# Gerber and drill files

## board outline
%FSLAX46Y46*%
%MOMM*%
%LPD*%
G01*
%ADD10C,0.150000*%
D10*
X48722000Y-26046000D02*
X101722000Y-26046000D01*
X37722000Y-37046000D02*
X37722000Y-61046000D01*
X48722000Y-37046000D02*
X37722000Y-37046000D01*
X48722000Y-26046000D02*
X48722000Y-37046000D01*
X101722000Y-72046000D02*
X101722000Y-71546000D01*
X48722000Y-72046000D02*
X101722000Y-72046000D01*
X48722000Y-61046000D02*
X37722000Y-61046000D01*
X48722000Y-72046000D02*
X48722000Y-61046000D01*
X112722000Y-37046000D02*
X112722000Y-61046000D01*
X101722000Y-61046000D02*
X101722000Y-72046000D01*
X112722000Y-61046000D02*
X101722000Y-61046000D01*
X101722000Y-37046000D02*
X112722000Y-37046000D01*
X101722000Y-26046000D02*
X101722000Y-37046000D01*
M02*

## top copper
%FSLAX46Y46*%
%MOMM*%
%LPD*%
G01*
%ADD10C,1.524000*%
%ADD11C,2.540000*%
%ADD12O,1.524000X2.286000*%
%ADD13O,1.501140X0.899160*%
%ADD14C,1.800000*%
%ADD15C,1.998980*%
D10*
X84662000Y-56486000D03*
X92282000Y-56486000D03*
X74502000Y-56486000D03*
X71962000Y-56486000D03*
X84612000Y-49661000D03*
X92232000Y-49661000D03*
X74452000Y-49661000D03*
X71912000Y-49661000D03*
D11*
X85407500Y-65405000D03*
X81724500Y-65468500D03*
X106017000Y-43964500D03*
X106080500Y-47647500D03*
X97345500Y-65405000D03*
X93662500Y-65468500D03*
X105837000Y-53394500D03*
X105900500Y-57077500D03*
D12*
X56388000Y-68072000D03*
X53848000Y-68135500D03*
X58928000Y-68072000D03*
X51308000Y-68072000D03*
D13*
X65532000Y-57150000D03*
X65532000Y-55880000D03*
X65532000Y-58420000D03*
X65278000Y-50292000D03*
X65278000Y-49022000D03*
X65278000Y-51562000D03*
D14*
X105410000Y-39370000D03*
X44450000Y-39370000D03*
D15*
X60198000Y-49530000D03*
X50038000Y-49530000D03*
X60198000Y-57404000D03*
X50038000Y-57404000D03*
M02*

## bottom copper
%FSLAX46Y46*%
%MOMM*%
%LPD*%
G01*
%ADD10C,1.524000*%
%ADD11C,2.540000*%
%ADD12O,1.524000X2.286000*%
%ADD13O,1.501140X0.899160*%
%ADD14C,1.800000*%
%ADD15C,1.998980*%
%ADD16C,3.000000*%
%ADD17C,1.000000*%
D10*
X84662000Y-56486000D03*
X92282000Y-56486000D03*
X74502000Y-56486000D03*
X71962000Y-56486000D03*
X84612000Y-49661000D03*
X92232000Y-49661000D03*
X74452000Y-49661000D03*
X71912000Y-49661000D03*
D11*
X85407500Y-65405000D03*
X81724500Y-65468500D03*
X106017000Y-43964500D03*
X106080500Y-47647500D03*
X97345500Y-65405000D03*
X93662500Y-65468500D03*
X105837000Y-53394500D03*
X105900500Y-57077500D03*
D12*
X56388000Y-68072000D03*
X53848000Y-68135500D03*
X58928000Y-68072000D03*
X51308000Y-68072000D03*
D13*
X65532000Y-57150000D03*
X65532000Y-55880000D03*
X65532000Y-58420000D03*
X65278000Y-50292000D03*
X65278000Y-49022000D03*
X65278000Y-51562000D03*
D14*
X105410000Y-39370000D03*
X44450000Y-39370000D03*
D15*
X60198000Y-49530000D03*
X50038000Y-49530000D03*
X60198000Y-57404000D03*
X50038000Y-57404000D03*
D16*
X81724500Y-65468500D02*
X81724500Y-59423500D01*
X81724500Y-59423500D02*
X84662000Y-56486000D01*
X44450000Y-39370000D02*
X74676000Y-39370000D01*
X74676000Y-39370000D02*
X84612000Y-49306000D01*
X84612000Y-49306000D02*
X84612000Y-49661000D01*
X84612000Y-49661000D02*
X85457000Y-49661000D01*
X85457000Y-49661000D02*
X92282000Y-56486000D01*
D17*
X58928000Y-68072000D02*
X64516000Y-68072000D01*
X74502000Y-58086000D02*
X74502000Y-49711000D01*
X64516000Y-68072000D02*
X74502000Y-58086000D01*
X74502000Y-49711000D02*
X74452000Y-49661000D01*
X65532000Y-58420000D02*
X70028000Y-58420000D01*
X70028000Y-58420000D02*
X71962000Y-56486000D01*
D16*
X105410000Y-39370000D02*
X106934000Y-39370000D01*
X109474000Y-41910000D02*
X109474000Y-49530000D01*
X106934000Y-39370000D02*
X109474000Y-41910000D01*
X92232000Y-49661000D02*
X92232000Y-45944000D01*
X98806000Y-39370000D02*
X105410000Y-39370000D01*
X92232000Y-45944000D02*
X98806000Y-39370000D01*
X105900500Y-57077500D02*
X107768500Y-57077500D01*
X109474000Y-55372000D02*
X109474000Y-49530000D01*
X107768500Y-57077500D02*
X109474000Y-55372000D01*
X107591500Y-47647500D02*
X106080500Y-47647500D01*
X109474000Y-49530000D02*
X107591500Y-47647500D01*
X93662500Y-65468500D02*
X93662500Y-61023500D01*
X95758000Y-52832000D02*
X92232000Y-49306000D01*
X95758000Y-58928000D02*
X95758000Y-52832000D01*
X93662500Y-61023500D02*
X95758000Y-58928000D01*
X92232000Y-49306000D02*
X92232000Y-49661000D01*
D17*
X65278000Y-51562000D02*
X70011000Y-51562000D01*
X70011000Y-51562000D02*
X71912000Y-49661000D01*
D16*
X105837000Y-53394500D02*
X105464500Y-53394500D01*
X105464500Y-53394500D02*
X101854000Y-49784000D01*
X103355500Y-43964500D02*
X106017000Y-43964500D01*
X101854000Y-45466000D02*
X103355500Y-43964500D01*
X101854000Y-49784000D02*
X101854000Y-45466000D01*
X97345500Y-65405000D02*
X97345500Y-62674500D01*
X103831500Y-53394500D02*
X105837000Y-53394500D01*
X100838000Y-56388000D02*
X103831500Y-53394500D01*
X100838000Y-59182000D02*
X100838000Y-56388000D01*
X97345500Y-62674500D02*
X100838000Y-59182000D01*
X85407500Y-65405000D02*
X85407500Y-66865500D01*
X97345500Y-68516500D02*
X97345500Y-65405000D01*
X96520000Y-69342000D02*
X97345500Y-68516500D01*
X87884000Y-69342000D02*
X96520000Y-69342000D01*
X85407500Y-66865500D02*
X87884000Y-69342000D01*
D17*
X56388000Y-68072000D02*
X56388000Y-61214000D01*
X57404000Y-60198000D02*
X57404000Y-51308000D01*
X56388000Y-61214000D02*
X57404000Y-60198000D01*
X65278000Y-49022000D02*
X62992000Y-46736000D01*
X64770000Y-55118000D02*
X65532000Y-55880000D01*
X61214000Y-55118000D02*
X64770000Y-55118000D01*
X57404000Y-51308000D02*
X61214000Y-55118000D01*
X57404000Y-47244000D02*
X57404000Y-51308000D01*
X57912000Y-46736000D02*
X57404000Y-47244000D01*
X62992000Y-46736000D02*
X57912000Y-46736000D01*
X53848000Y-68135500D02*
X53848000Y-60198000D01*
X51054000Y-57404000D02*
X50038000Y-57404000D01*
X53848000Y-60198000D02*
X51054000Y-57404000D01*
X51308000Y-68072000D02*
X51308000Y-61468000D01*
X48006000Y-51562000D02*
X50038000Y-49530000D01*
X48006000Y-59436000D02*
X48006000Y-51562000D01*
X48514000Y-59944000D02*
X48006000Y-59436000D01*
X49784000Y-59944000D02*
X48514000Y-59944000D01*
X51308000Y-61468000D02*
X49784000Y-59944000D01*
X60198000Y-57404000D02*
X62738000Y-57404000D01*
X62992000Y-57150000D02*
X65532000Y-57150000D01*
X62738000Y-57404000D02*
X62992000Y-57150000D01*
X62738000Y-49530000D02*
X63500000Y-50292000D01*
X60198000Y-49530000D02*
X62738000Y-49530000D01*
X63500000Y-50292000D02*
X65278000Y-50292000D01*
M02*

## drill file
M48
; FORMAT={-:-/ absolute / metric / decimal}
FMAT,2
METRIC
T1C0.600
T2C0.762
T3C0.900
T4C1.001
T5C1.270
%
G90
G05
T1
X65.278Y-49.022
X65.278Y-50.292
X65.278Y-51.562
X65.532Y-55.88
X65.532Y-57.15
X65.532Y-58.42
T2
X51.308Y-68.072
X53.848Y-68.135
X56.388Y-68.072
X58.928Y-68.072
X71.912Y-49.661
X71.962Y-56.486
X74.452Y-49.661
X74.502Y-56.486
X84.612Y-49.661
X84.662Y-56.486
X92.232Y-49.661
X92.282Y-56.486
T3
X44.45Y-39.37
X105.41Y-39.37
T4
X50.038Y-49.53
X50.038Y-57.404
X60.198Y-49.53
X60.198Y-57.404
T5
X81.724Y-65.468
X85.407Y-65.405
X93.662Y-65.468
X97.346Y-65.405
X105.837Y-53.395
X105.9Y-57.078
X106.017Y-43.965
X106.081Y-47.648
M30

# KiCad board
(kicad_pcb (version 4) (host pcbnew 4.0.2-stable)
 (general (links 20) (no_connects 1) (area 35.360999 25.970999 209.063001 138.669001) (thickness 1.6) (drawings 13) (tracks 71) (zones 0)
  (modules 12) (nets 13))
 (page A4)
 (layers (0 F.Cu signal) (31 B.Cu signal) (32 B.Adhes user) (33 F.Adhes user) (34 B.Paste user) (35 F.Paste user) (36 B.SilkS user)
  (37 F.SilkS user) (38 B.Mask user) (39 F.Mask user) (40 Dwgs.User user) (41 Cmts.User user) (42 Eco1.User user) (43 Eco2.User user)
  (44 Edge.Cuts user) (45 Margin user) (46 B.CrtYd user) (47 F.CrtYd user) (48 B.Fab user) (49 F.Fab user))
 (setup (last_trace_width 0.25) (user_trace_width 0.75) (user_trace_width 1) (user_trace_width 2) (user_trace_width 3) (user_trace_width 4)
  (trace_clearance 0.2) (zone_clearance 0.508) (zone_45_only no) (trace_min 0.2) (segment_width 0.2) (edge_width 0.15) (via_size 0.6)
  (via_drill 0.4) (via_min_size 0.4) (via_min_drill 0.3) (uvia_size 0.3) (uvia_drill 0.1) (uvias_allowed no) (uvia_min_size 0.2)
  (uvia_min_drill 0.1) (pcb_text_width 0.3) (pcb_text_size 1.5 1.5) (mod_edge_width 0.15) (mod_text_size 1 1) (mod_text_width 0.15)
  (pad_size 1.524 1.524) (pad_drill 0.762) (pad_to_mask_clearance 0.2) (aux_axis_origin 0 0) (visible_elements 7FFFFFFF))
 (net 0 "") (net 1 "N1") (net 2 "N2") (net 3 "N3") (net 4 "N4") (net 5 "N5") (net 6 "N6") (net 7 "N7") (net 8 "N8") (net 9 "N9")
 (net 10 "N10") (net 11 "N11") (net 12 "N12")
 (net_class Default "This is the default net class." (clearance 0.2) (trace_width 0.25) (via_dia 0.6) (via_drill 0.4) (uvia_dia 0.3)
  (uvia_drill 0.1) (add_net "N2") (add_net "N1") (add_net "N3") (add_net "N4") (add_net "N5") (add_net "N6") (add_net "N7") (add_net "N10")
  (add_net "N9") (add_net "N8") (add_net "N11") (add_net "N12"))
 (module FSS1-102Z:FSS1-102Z (layer F.Cu) (at 82.122 57.121 180)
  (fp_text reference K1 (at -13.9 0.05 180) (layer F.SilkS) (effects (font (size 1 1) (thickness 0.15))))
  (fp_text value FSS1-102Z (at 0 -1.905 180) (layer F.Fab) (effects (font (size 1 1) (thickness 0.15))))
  (pad 2 thru_hole circle (at -2.54 0.635 180) (size 1.524 1.524) (drill 0.762) (layers *.Cu *.Mask F.SilkS) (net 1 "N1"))
  (pad 1 thru_hole circle (at -10.16 0.635 180) (size 1.524 1.524) (drill 0.762) (layers *.Cu *.Mask F.SilkS) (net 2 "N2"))
  (pad 3 thru_hole circle (at 7.62 0.635 180) (size 1.524 1.524) (drill 0.762) (layers *.Cu *.Mask F.SilkS) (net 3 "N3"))
  (pad 4 thru_hole circle (at 10.16 0.635 180) (size 1.524 1.524) (drill 0.762) (layers *.Cu *.Mask F.SilkS) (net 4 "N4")))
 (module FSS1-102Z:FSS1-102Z (layer F.Cu) (at 82.072 50.296 180)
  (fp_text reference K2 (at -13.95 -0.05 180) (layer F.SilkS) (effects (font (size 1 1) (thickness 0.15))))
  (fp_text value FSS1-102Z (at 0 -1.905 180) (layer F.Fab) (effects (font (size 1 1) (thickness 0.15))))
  (pad 2 thru_hole circle (at -2.54 0.635 180) (size 1.524 1.524) (drill 0.762) (layers *.Cu *.Mask F.SilkS) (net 2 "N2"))
  (pad 1 thru_hole circle (at -10.16 0.635 180) (size 1.524 1.524) (drill 0.762) (layers *.Cu *.Mask F.SilkS) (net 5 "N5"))
  (pad 3 thru_hole circle (at 7.62 0.635 180) (size 1.524 1.524) (drill 0.762) (layers *.Cu *.Mask F.SilkS) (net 3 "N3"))
  (pad 4 thru_hole circle (at 10.16 0.635 180) (size 1.524 1.524) (drill 0.762) (layers *.Cu *.Mask F.SilkS) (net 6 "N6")))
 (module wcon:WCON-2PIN (layer F.Cu) (at 83.566 66.04)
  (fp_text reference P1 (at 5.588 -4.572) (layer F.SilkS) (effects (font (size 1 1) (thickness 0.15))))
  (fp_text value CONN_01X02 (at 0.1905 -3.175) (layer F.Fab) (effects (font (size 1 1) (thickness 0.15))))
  (pad 2 thru_hole circle (at 1.8415 -0.635) (size 2.54 2.54) (drill 1.27) (layers *.Cu *.Mask F.SilkS) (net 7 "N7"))
  (pad 1 thru_hole circle (at -1.8415 -0.5715) (size 2.54 2.54) (drill 1.27) (layers *.Cu *.Mask F.SilkS) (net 1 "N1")))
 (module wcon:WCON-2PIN (layer F.Cu) (at 106.652 45.806 90)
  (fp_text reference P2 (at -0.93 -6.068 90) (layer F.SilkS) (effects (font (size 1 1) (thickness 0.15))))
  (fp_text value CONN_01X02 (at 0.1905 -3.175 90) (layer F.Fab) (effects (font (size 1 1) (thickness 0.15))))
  (pad 2 thru_hole circle (at 1.8415 -0.635 90) (size 2.54 2.54) (drill 1.27) (layers *.Cu *.Mask F.SilkS) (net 7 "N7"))
  (pad 1 thru_hole circle (at -1.8415 -0.5715 90) (size 2.54 2.54) (drill 1.27) (layers *.Cu *.Mask F.SilkS) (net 5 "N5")))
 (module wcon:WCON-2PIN (layer F.Cu) (at 95.504 66.04)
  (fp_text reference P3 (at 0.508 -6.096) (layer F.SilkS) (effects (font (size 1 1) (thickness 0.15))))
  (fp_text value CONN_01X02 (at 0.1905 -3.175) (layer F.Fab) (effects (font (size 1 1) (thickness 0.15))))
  (pad 2 thru_hole circle (at 1.8415 -0.635) (size 2.54 2.54) (drill 1.27) (layers *.Cu *.Mask F.SilkS) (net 7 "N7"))
  (pad 1 thru_hole circle (at -1.8415 -0.5715) (size 2.54 2.54) (drill 1.27) (layers *.Cu *.Mask F.SilkS) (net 5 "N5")))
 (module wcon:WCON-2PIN (layer F.Cu) (at 106.472 55.236 90)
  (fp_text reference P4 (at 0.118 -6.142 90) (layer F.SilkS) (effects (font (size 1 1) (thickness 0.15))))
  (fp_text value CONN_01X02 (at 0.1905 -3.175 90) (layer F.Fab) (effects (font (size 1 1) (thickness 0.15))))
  (pad 2 thru_hole circle (at 1.8415 -0.635 90) (size 2.54 2.54) (drill 1.27) (layers *.Cu *.Mask F.SilkS) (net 7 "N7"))
  (pad 1 thru_hole circle (at -1.8415 -0.5715 90) (size 2.54 2.54) (drill 1.27) (layers *.Cu *.Mask F.SilkS) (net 5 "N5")))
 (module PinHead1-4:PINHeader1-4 (layer F.Cu) (at 55.118 68.072)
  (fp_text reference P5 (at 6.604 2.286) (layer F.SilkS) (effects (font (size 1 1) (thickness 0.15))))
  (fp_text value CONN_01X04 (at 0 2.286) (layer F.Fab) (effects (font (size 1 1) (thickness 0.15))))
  (pad 3 thru_hole oval (at 1.27 0) (size 1.524 2.286) (drill 0.762) (layers *.Cu *.Mask F.SilkS) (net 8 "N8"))
  (pad 2 thru_hole oval (at -1.27 0.0635) (size 1.524 2.286) (drill 0.762) (layers *.Cu *.Mask F.SilkS) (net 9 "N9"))
  (pad 4 thru_hole oval (at 3.81 0) (size 1.524 2.286) (drill 0.762) (layers *.Cu *.Mask F.SilkS) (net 3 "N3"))
  (pad 1 thru_hole oval (at -3.81 0) (size 1.524 2.286) (drill 0.762) (layers *.Cu *.Mask F.SilkS) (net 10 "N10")))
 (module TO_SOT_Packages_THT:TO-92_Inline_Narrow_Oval (layer F.Cu) (at 65.532 58.42 90)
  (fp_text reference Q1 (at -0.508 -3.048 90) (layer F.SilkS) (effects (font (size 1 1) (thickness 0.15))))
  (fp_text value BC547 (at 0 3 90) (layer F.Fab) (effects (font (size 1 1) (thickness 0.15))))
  (pad 2 thru_hole oval (at 1.27 0 270) (size 0.89916 1.50114) (drill 0.6) (layers *.Cu *.Mask F.SilkS) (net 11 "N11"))
  (pad 3 thru_hole oval (at 2.54 0 270) (size 0.89916 1.50114) (drill 0.6) (layers *.Cu *.Mask F.SilkS) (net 8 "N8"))
  (pad 1 thru_hole oval (at 0 0 270) (size 0.89916 1.50114) (drill 0.6) (layers *.Cu *.Mask F.SilkS) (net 4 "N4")))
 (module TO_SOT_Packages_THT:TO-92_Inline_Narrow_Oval (layer F.Cu) (at 65.278 51.562 90)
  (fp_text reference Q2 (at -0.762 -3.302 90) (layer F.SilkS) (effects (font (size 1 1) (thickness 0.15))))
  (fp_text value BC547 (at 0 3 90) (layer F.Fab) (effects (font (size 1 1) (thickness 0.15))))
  (pad 2 thru_hole oval (at 1.27 0 270) (size 0.89916 1.50114) (drill 0.6) (layers *.Cu *.Mask F.SilkS) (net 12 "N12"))
  (pad 3 thru_hole oval (at 2.54 0 270) (size 0.89916 1.50114) (drill 0.6) (layers *.Cu *.Mask F.SilkS) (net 8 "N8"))
  (pad 1 thru_hole oval (at 0 0 270) (size 0.89916 1.50114) (drill 0.6) (layers *.Cu *.Mask F.SilkS) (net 6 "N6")))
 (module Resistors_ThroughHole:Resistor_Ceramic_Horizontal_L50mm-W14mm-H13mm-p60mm (layer F.Cu) (at 74.93 39.37 180)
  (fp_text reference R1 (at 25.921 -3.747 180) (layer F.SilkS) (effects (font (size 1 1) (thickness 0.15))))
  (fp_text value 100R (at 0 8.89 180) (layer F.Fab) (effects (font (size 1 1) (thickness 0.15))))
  (pad 1 thru_hole circle (at -30.48 0) (size 1.8 1.8) (drill 0.9) (layers *.Cu *.Mask F.SilkS) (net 5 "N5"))
  (pad 2 thru_hole circle (at 30.48 0) (size 1.8 1.8) (drill 0.9) (layers *.Cu *.Mask F.SilkS) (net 2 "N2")))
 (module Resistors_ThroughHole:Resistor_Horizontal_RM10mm (layer F.Cu) (at 60.198 49.53 180)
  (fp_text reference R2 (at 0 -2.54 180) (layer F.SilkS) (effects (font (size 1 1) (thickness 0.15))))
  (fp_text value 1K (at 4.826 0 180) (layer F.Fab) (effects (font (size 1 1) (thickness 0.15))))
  (pad 1 thru_hole circle (at 0 0 180) (size 1.99898 1.99898) (drill 1.00076) (layers *.Cu *.SilkS *.Mask) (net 12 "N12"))
  (pad 2 thru_hole circle (at 10.16 0 180) (size 1.99898 1.99898) (drill 1.00076) (layers *.Cu *.SilkS *.Mask) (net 10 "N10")))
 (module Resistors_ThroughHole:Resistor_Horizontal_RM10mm (layer F.Cu) (at 60.198 57.404 180)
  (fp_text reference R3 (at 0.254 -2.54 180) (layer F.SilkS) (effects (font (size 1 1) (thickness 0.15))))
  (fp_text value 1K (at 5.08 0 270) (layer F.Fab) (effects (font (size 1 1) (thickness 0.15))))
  (pad 1 thru_hole circle (at 0 0 180) (size 1.99898 1.99898) (drill 1.00076) (layers *.Cu *.SilkS *.Mask) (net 11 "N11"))
  (pad 2 thru_hole circle (at 10.16 0 180) (size 1.99898 1.99898) (drill 1.00076) (layers *.Cu *.SilkS *.Mask) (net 9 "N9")))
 (gr_line (start 48.722 26.046) (end 101.722 26.046) (angle 90) (layer Edge.Cuts) (width 0.15))
 (gr_line (start 37.722 37.046) (end 37.722 61.046) (angle 90) (layer Edge.Cuts) (width 0.15))
 (gr_line (start 48.722 37.046) (end 37.722 37.046) (angle 90) (layer Edge.Cuts) (width 0.15))
 (gr_line (start 48.722 26.046) (end 48.722 37.046) (angle 90) (layer Edge.Cuts) (width 0.15))
 (gr_line (start 101.722 72.046) (end 101.722 71.546) (angle 90) (layer Edge.Cuts) (width 0.15))
 (gr_line (start 48.722 72.046) (end 101.722 72.046) (angle 90) (layer Edge.Cuts) (width 0.15))
 (gr_line (start 48.722 61.046) (end 37.722 61.046) (angle 90) (layer Edge.Cuts) (width 0.15))
 (gr_line (start 48.722 72.046) (end 48.722 61.046) (angle 90) (layer Edge.Cuts) (width 0.15))
 (gr_line (start 112.722 37.046) (end 112.722 61.046) (angle 90) (layer Edge.Cuts) (width 0.15))
 (gr_line (start 101.722 61.046) (end 101.722 72.046) (angle 90) (layer Edge.Cuts) (width 0.15))
 (gr_line (start 112.722 61.046) (end 101.722 61.046) (angle 90) (layer Edge.Cuts) (width 0.15))
 (gr_line (start 101.722 37.046) (end 112.722 37.046) (angle 90) (layer Edge.Cuts) (width 0.15))
 (gr_line (start 101.722 26.046) (end 101.722 37.046) (angle 90) (layer Edge.Cuts) (width 0.15))
 (segment (start 81.7245 65.4685) (end 81.7245 59.4235) (width 3) (layer B.Cu) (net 1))
 (segment (start 81.7245 59.4235) (end 84.662 56.486) (width 3) (layer B.Cu) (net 1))
 (segment (start 44.45 39.37) (end 74.676 39.37) (width 3) (layer B.Cu) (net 2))
 (segment (start 74.676 39.37) (end 84.612 49.306) (width 3) (layer B.Cu) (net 2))
 (segment (start 84.612 49.306) (end 84.612 49.661) (width 3) (layer B.Cu) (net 2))
 (segment (start 84.612 49.661) (end 85.457 49.661) (width 3) (layer B.Cu) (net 2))
 (segment (start 85.457 49.661) (end 92.282 56.486) (width 3) (layer B.Cu) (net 2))
 (segment (start 58.928 68.072) (end 64.516 68.072) (width 1) (layer B.Cu) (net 3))
 (segment (start 74.502 58.086) (end 74.502 49.711) (width 1) (layer B.Cu) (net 3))
 (segment (start 64.516 68.072) (end 74.502 58.086) (width 1) (layer B.Cu) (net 3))
 (segment (start 74.502 49.711) (end 74.452 49.661) (width 1) (layer B.Cu) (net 3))
 (segment (start 65.532 58.42) (end 70.028 58.42) (width 1) (layer B.Cu) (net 4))
 (segment (start 70.028 58.42) (end 71.962 56.486) (width 1) (layer B.Cu) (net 4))
 (segment (start 105.41 39.37) (end 106.934 39.37) (width 3) (layer B.Cu) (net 5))
 (segment (start 109.474 41.91) (end 109.474 49.53) (width 3) (layer B.Cu) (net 5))
 (segment (start 106.934 39.37) (end 109.474 41.91) (width 3) (layer B.Cu) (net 5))
 (segment (start 92.232 49.661) (end 92.232 45.944) (width 3) (layer B.Cu) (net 5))
 (segment (start 98.806 39.37) (end 105.41 39.37) (width 3) (layer B.Cu) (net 5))
 (segment (start 92.232 45.944) (end 98.806 39.37) (width 3) (layer B.Cu) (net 5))
 (segment (start 105.9005 57.0775) (end 107.7685 57.0775) (width 3) (layer B.Cu) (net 5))
 (segment (start 109.474 55.372) (end 109.474 49.53) (width 3) (layer B.Cu) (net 5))
 (segment (start 107.7685 57.0775) (end 109.474 55.372) (width 3) (layer B.Cu) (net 5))
 (segment (start 107.5915 47.6475) (end 106.0805 47.6475) (width 3) (layer B.Cu) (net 5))
 (segment (start 109.474 49.53) (end 107.5915 47.6475) (width 3) (layer B.Cu) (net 5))
 (segment (start 93.6625 65.4685) (end 93.6625 61.0235) (width 3) (layer B.Cu) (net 5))
 (segment (start 95.758 52.832) (end 92.232 49.306) (width 3) (layer B.Cu) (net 5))
 (segment (start 95.758 58.928) (end 95.758 52.832) (width 3) (layer B.Cu) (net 5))
 (segment (start 93.6625 61.0235) (end 95.758 58.928) (width 3) (layer B.Cu) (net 5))
 (segment (start 92.232 49.306) (end 92.232 49.661) (width 3) (layer B.Cu) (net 5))
 (segment (start 65.278 51.562) (end 70.011 51.562) (width 1) (layer B.Cu) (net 6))
 (segment (start 70.011 51.562) (end 71.912 49.661) (width 1) (layer B.Cu) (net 6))
 (segment (start 105.837 53.3945) (end 105.4645 53.3945) (width 3) (layer B.Cu) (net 7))
 (segment (start 105.4645 53.3945) (end 101.854 49.784) (width 3) (layer B.Cu) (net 7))
 (segment (start 103.3555 43.9645) (end 106.017 43.9645) (width 3) (layer B.Cu) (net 7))
 (segment (start 101.854 45.466) (end 103.3555 43.9645) (width 3) (layer B.Cu) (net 7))
 (segment (start 101.854 49.784) (end 101.854 45.466) (width 3) (layer B.Cu) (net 7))
 (segment (start 97.3455 65.405) (end 97.3455 62.6745) (width 3) (layer B.Cu) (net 7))
 (segment (start 103.8315 53.3945) (end 105.837 53.3945) (width 3) (layer B.Cu) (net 7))
 (segment (start 100.838 56.388) (end 103.8315 53.3945) (width 3) (layer B.Cu) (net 7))
 (segment (start 100.838 59.182) (end 100.838 56.388) (width 3) (layer B.Cu) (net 7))
 (segment (start 97.3455 62.6745) (end 100.838 59.182) (width 3) (layer B.Cu) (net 7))
 (segment (start 85.4075 65.405) (end 85.4075 66.8655) (width 3) (layer B.Cu) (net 7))
 (segment (start 97.3455 68.5165) (end 97.3455 65.405) (width 3) (layer B.Cu) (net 7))
 (segment (start 96.52 69.342) (end 97.3455 68.5165) (width 3) (layer B.Cu) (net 7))
 (segment (start 87.884 69.342) (end 96.52 69.342) (width 3) (layer B.Cu) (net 7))
 (segment (start 85.4075 66.8655) (end 87.884 69.342) (width 3) (layer B.Cu) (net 7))
 (segment (start 56.388 68.072) (end 56.388 61.214) (width 1) (layer B.Cu) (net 8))
 (segment (start 57.404 60.198) (end 57.404 51.308) (width 1) (layer B.Cu) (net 8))
 (segment (start 56.388 61.214) (end 57.404 60.198) (width 1) (layer B.Cu) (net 8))
 (segment (start 65.278 49.022) (end 62.992 46.736) (width 1) (layer B.Cu) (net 8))
 (segment (start 64.77 55.118) (end 65.532 55.88) (width 1) (layer B.Cu) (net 8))
 (segment (start 61.214 55.118) (end 64.77 55.118) (width 1) (layer B.Cu) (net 8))
 (segment (start 57.404 51.308) (end 61.214 55.118) (width 1) (layer B.Cu) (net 8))
 (segment (start 57.404 47.244) (end 57.404 51.308) (width 1) (layer B.Cu) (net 8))
 (segment (start 57.912 46.736) (end 57.404 47.244) (width 1) (layer B.Cu) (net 8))
 (segment (start 62.992 46.736) (end 57.912 46.736) (width 1) (layer B.Cu) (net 8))
 (segment (start 53.848 68.1355) (end 53.848 60.198) (width 1) (layer B.Cu) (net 9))
 (segment (start 51.054 57.404) (end 50.038 57.404) (width 1) (layer B.Cu) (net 9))
 (segment (start 53.848 60.198) (end 51.054 57.404) (width 1) (layer B.Cu) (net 9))
 (segment (start 51.308 68.072) (end 51.308 61.468) (width 1) (layer B.Cu) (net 10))
 (segment (start 48.006 51.562) (end 50.038 49.53) (width 1) (layer B.Cu) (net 10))
 (segment (start 48.006 59.436) (end 48.006 51.562) (width 1) (layer B.Cu) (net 10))
 (segment (start 48.514 59.944) (end 48.006 59.436) (width 1) (layer B.Cu) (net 10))
 (segment (start 49.784 59.944) (end 48.514 59.944) (width 1) (layer B.Cu) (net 10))
 (segment (start 51.308 61.468) (end 49.784 59.944) (width 1) (layer B.Cu) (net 10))
 (segment (start 60.198 57.404) (end 62.738 57.404) (width 1) (layer B.Cu) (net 11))
 (segment (start 62.992 57.15) (end 65.532 57.15) (width 1) (layer B.Cu) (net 11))
 (segment (start 62.738 57.404) (end 62.992 57.15) (width 1) (layer B.Cu) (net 11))
 (segment (start 62.738 49.53) (end 63.5 50.292) (width 1) (layer B.Cu) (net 12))
 (segment (start 60.198 49.53) (end 62.738 49.53) (width 1) (layer B.Cu) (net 12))
 (segment (start 63.5 50.292) (end 65.278 50.292) (width 1) (layer B.Cu) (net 12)))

